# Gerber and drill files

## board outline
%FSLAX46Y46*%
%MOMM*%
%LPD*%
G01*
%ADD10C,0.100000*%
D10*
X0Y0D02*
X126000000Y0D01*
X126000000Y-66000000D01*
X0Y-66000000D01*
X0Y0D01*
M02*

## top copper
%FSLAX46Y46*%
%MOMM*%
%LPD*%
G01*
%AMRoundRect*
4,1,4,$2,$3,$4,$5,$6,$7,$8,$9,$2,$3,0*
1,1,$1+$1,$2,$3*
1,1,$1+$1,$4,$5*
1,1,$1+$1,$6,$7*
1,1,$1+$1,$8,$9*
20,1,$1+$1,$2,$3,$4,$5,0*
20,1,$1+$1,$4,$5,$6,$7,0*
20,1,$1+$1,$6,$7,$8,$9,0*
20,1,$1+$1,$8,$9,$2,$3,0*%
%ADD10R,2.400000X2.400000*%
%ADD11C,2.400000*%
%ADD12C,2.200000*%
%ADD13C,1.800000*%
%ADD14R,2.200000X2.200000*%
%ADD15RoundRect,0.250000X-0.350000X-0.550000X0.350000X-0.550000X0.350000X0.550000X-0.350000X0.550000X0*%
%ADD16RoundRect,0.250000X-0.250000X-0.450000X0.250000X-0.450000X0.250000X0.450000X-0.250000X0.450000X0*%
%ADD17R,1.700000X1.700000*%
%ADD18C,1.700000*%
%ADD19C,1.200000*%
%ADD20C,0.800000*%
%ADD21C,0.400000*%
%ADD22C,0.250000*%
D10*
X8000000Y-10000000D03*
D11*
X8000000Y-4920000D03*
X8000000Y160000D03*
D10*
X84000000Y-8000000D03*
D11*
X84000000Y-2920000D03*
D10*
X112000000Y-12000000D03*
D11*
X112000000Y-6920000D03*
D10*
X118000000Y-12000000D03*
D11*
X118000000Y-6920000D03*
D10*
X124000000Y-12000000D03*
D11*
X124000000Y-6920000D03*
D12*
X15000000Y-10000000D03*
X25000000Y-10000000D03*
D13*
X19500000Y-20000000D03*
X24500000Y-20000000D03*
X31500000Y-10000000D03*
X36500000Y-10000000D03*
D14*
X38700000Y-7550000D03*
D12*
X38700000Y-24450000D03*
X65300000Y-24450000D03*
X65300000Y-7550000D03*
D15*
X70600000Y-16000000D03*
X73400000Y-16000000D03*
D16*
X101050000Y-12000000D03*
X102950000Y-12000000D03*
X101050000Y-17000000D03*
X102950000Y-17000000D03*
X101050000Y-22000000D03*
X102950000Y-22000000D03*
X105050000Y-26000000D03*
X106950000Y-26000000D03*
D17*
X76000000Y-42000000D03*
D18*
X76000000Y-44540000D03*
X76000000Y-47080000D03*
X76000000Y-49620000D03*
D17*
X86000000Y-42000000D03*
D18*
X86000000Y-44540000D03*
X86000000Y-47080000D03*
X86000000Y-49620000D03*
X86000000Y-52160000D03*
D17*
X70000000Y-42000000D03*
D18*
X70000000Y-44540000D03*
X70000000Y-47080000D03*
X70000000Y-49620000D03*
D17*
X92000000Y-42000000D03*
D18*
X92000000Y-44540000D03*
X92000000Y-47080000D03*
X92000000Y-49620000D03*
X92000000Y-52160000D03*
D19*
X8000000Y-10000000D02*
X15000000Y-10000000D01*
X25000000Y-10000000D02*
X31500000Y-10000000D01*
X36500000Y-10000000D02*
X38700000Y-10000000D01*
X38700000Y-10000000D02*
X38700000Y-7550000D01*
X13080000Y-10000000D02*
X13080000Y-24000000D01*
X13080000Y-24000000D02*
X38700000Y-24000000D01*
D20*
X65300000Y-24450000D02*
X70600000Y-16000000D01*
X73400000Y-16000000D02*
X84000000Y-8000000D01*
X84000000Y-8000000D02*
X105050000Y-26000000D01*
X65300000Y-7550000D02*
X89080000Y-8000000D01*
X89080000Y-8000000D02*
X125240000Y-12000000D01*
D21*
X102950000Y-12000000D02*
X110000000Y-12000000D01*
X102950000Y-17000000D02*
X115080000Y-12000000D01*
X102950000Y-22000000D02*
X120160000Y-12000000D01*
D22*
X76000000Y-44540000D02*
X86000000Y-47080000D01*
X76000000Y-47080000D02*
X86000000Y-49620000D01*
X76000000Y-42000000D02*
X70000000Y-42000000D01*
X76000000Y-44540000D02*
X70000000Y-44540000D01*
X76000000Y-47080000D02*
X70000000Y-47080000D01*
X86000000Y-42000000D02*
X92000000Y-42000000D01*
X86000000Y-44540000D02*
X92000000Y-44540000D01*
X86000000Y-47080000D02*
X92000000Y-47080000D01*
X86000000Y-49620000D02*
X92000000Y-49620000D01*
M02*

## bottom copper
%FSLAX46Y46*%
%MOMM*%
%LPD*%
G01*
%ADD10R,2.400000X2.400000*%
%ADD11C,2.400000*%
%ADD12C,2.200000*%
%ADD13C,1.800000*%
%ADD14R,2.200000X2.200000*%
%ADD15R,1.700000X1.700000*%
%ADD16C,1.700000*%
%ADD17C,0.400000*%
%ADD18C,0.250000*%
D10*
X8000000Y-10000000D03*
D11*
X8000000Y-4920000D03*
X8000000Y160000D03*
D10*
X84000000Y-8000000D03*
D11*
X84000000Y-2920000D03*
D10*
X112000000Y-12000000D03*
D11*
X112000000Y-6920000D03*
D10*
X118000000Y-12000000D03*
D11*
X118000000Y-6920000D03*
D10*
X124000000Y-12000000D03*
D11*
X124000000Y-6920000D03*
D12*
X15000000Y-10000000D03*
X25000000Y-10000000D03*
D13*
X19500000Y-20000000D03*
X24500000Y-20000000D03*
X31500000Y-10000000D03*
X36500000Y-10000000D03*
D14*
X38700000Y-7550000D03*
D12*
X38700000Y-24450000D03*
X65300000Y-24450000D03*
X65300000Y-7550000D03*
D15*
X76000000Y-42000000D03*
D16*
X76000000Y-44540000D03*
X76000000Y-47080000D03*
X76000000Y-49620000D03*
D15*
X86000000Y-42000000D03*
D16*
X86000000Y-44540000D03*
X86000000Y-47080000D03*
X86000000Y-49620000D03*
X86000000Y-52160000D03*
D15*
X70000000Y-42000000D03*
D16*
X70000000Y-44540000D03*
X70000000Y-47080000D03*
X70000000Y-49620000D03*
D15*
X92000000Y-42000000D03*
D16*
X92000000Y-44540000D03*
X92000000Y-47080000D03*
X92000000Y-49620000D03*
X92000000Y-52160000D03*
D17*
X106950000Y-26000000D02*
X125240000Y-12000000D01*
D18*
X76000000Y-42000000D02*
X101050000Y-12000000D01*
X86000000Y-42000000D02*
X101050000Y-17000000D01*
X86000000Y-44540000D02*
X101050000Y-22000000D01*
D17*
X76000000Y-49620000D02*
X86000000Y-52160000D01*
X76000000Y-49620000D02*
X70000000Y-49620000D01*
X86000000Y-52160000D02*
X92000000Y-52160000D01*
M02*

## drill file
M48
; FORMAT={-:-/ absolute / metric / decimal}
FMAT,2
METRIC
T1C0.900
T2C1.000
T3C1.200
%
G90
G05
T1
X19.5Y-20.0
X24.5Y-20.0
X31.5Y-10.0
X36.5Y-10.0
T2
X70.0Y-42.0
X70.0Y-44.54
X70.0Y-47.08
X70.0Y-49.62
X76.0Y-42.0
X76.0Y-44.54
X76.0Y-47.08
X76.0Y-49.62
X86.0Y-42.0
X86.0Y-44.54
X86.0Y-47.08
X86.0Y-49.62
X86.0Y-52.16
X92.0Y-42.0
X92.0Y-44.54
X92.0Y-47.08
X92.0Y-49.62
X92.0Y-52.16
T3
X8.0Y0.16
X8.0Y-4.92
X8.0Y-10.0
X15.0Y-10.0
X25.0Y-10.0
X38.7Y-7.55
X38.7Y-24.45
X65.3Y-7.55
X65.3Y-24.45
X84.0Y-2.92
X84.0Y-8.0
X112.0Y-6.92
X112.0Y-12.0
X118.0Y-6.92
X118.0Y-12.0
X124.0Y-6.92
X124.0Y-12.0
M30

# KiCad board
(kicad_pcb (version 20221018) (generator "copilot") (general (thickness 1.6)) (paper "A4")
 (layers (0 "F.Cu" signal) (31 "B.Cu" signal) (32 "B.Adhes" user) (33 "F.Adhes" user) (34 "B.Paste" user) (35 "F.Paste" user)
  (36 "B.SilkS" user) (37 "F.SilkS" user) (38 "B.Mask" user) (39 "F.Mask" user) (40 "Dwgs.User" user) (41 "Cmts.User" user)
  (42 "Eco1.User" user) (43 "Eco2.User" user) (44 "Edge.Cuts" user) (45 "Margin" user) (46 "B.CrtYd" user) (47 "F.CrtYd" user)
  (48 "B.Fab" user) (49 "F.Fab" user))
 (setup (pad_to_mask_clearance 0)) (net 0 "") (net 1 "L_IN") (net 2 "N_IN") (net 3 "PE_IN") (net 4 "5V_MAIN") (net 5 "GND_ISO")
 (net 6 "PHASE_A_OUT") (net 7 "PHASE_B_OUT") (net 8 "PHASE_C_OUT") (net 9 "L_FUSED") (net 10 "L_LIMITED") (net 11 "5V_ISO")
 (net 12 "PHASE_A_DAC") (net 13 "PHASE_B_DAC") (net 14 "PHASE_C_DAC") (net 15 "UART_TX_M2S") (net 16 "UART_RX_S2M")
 (gr_rect (start 0 0) (end 126 66) (stroke (width 0.1) (type solid)) (fill none) (layer "Edge.Cuts"))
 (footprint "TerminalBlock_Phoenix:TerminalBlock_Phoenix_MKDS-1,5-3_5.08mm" (layer "F.Cu") (at 8 10 90)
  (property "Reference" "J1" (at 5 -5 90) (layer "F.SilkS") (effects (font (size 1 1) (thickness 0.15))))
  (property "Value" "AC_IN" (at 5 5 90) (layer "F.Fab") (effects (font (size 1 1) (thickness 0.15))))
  (pad "1" thru_hole rect (at 0 0 90) (size 2.4 2.4) (drill 1.2) (layers "*.Cu" "*.Mask") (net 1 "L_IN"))
  (pad "2" thru_hole circle (at 5.08 0 90) (size 2.4 2.4) (drill 1.2) (layers "*.Cu" "*.Mask") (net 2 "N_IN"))
  (pad "3" thru_hole circle (at 10.16 0 90) (size 2.4 2.4) (drill 1.2) (layers "*.Cu" "*.Mask") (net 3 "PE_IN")))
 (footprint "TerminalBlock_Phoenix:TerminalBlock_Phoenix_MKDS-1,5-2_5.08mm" (layer "F.Cu") (at 84 8 90)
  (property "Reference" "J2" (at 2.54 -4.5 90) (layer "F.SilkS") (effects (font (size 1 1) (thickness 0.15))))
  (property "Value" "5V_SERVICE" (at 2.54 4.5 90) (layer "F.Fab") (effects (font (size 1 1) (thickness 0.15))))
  (pad "1" thru_hole rect (at 0 0 90) (size 2.4 2.4) (drill 1.2) (layers "*.Cu" "*.Mask") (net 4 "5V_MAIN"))
  (pad "2" thru_hole circle (at 5.08 0 90) (size 2.4 2.4) (drill 1.2) (layers "*.Cu" "*.Mask") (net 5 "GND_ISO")))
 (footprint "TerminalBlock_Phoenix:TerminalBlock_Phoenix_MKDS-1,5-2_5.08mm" (layer "F.Cu") (at 112 12 90)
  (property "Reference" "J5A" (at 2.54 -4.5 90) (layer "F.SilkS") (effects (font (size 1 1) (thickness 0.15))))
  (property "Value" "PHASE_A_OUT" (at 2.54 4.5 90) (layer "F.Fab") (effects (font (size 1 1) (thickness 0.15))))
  (pad "1" thru_hole rect (at 0 0 90) (size 2.4 2.4) (drill 1.2) (layers "*.Cu" "*.Mask") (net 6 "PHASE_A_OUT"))
  (pad "2" thru_hole circle (at 5.08 0 90) (size 2.4 2.4) (drill 1.2) (layers "*.Cu" "*.Mask") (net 5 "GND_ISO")))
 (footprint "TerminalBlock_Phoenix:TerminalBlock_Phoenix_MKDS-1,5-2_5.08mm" (layer "F.Cu") (at 118 12 90)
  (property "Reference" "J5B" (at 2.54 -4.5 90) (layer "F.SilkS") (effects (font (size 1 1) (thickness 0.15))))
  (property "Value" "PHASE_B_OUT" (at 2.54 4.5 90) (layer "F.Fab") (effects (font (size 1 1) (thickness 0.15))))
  (pad "1" thru_hole rect (at 0 0 90) (size 2.4 2.4) (drill 1.2) (layers "*.Cu" "*.Mask") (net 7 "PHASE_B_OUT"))
  (pad "2" thru_hole circle (at 5.08 0 90) (size 2.4 2.4) (drill 1.2) (layers "*.Cu" "*.Mask") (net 5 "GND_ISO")))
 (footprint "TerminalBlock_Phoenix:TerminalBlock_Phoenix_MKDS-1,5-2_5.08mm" (layer "F.Cu") (at 124 12 90)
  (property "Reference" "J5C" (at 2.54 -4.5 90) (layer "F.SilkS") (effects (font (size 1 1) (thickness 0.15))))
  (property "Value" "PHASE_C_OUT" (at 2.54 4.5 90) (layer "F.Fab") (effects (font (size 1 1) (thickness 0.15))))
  (pad "1" thru_hole rect (at 0 0 90) (size 2.4 2.4) (drill 1.2) (layers "*.Cu" "*.Mask") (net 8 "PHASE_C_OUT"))
  (pad "2" thru_hole circle (at 5.08 0 90) (size 2.4 2.4) (drill 1.2) (layers "*.Cu" "*.Mask") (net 5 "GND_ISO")))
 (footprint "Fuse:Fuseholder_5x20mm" (layer "F.Cu") (at 20 10 0)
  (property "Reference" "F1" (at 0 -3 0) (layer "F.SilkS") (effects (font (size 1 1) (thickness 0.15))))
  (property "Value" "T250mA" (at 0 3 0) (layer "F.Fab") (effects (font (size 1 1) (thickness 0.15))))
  (pad "1" thru_hole circle (at -5 0 0) (size 2.2 2.2) (drill 1.2) (layers "*.Cu" "*.Mask") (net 1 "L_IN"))
  (pad "2" thru_hole circle (at 5 0 0) (size 2.2 2.2) (drill 1.2) (layers "*.Cu" "*.Mask") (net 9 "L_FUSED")))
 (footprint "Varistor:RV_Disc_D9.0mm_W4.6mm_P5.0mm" (layer "F.Cu") (at 22 20 0)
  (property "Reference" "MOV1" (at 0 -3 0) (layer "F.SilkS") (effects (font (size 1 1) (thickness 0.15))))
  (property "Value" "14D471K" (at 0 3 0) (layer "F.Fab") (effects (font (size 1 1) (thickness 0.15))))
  (pad "1" thru_hole circle (at -2.5 0 0) (size 1.8 1.8) (drill 0.9) (layers "*.Cu" "*.Mask") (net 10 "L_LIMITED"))
  (pad "2" thru_hole circle (at 2.5 0 0) (size 1.8 1.8) (drill 0.9) (layers "*.Cu" "*.Mask") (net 2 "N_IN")))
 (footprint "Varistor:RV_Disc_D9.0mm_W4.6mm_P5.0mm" (layer "F.Cu") (at 34 10 0)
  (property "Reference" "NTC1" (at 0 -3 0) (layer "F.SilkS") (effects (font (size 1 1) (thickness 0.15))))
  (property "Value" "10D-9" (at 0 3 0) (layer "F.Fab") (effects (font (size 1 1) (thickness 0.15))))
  (pad "1" thru_hole circle (at -2.5 0 0) (size 1.8 1.8) (drill 0.9) (layers "*.Cu" "*.Mask") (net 9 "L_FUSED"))
  (pad "2" thru_hole circle (at 2.5 0 0) (size 1.8 1.8) (drill 0.9) (layers "*.Cu" "*.Mask") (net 10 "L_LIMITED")))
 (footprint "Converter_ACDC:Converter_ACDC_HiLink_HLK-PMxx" (layer "F.Cu") (at 52 16 0)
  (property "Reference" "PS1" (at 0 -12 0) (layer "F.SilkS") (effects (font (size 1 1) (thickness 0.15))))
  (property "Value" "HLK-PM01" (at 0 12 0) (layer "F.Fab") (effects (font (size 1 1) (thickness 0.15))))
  (pad "1" thru_hole rect (at -13.3 -8.45 0) (size 2.2 2.2) (drill 1.2) (layers "*.Cu" "*.Mask") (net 10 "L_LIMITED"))
  (pad "2" thru_hole circle (at -13.3 8.45 0) (size 2.2 2.2) (drill 1.2) (layers "*.Cu" "*.Mask") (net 2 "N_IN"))
  (pad "3" thru_hole circle (at 13.3 8.45 0) (size 2.2 2.2) (drill 1.2) (layers "*.Cu" "*.Mask") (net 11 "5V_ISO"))
  (pad "4" thru_hole circle (at 13.3 -8.45 0) (size 2.2 2.2) (drill 1.2) (layers "*.Cu" "*.Mask") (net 5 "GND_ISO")))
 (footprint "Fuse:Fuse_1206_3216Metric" (layer "F.Cu") (at 72 16 0)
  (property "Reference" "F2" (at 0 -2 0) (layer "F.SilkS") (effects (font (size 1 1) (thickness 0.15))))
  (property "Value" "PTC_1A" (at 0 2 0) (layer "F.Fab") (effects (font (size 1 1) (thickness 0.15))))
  (pad "1" smd roundrect (at -1.4 0 0) (size 1.2 1.6) (layers "F.Cu" "F.Paste" "F.Mask") (roundrect_rratio 0.208333) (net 11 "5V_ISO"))
  (pad "2" smd roundrect (at 1.4 0 0) (size 1.2 1.6) (layers "F.Cu" "F.Paste" "F.Mask") (roundrect_rratio 0.208333) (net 4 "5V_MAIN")))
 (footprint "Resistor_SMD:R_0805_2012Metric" (layer "F.Cu") (at 102 12 0)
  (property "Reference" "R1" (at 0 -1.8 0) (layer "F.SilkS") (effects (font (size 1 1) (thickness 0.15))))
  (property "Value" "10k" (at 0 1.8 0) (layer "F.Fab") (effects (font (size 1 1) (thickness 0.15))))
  (pad "1" smd roundrect (at -0.95 0 0) (size 1 1.4) (layers "F.Cu" "F.Paste" "F.Mask") (roundrect_rratio 0.25) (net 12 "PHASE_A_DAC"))
  (pad "2" smd roundrect (at 0.95 0 0) (size 1 1.4) (layers "F.Cu" "F.Paste" "F.Mask") (roundrect_rratio 0.25) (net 6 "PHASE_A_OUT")))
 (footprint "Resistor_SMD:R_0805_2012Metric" (layer "F.Cu") (at 102 17 0)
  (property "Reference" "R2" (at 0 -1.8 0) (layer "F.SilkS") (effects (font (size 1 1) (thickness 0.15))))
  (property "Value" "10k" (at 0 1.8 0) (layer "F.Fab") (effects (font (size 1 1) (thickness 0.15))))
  (pad "1" smd roundrect (at -0.95 0 0) (size 1 1.4) (layers "F.Cu" "F.Paste" "F.Mask") (roundrect_rratio 0.25) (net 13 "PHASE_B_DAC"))
  (pad "2" smd roundrect (at 0.95 0 0) (size 1 1.4) (layers "F.Cu" "F.Paste" "F.Mask") (roundrect_rratio 0.25) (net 7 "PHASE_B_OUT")))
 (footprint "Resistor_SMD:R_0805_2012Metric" (layer "F.Cu") (at 102 22 0)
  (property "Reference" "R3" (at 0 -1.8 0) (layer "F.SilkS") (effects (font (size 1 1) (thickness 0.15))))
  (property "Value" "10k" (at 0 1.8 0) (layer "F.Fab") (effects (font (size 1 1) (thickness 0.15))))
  (pad "1" smd roundrect (at -0.95 0 0) (size 1 1.4) (layers "F.Cu" "F.Paste" "F.Mask") (roundrect_rratio 0.25) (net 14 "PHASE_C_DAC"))
  (pad "2" smd roundrect (at 0.95 0 0) (size 1 1.4) (layers "F.Cu" "F.Paste" "F.Mask") (roundrect_rratio 0.25) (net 8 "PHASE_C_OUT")))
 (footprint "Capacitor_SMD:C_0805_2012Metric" (layer "F.Cu") (at 106 26 0)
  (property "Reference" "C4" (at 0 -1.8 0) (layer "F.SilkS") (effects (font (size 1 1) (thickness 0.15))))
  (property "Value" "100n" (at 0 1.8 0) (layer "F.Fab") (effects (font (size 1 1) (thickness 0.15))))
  (pad "1" smd roundrect (at -0.95 0 0) (size 1 1.4) (layers "F.Cu" "F.Paste" "F.Mask") (roundrect_rratio 0.25) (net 4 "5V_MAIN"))
  (pad "2" smd roundrect (at 0.95 0 0) (size 1 1.4) (layers "F.Cu" "F.Paste" "F.Mask") (roundrect_rratio 0.25) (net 5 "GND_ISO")))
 (segment (start 8 10) (end 15 10) (width 1.2) (layer "F.Cu") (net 1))
 (segment (start 25 10) (end 31.5 10) (width 1.2) (layer "F.Cu") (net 9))
 (segment (start 36.5 10) (end 38.7 10) (width 1.2) (layer "F.Cu") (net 10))
 (segment (start 38.7 10) (end 38.7 7.55) (width 1.2) (layer "F.Cu") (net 10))
 (segment (start 13.08 10) (end 13.08 24) (width 1.2) (layer "F.Cu") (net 2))
 (segment (start 13.08 24) (end 38.7 24) (width 1.2) (layer "F.Cu") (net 2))
 (segment (start 65.3 24.45) (end 70.6 16) (width 0.8) (layer "F.Cu") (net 11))
 (segment (start 73.4 16) (end 84 8) (width 0.8) (layer "F.Cu") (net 4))
 (segment (start 84 8) (end 105.05 26) (width 0.8) (layer "F.Cu") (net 4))
 (segment (start 65.3 7.55) (end 89.08 8) (width 0.8) (layer "F.Cu") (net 5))
 (segment (start 89.08 8) (end 125.24 12) (width 0.8) (layer "F.Cu") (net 5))
 (segment (start 106.95 26) (end 125.24 12) (width 0.4) (layer "B.Cu") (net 5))
 (segment (start 102.95 12) (end 110 12) (width 0.4) (layer "F.Cu") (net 6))
 (segment (start 102.95 17) (end 115.08 12) (width 0.4) (layer "F.Cu") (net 7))
 (segment (start 102.95 22) (end 120.16 12) (width 0.4) (layer "F.Cu") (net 8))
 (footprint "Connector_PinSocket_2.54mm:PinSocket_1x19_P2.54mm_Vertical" (layer "F.Cu") (at 28 46 0)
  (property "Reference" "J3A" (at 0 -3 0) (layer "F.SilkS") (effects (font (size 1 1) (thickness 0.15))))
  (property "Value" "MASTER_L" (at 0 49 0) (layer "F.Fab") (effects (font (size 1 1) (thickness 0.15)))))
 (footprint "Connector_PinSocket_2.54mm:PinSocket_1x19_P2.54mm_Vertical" (layer "F.Cu") (at 36 46 0)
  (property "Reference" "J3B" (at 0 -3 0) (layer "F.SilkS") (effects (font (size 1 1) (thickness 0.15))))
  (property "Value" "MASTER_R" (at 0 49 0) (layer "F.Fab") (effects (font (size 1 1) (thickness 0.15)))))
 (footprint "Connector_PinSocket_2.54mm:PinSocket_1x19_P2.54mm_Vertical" (layer "F.Cu") (at 92 46 0)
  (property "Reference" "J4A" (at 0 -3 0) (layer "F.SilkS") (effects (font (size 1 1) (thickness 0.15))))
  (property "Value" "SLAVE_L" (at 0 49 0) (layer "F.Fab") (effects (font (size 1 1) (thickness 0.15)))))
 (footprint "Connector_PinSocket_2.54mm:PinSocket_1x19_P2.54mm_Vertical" (layer "F.Cu") (at 100 46 0)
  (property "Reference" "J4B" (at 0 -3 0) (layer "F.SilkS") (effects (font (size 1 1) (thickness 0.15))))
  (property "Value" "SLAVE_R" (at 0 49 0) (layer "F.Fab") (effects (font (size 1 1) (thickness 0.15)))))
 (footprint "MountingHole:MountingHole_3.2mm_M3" (layer "F.Cu") (at 5 5)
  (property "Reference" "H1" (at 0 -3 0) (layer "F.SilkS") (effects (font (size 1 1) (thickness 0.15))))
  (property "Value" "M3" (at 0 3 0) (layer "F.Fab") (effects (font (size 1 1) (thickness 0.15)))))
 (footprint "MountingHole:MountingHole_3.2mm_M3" (layer "F.Cu") (at 121 5)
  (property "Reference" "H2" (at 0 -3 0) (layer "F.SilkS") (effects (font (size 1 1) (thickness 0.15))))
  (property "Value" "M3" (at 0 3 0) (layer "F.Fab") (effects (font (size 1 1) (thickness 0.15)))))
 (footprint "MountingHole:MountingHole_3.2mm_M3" (layer "F.Cu") (at 5 61)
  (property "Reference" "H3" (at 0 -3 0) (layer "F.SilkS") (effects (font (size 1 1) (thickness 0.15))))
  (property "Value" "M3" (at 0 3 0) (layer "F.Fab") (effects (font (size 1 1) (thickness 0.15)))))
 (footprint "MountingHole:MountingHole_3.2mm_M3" (layer "F.Cu") (at 121 61)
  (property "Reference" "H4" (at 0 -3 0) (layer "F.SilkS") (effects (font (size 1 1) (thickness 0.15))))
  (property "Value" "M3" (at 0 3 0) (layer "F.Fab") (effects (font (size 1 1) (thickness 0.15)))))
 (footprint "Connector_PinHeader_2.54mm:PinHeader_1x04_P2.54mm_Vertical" (layer "F.Cu") (at 76 42 0)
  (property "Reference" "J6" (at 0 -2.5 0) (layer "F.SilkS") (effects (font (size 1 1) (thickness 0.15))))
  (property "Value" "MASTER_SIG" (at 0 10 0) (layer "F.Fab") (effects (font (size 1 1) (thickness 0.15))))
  (pad "1" thru_hole rect (at 0 0 0) (size 1.7 1.7) (drill 1) (layers "*.Cu" "*.Mask") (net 12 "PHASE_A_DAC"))
  (pad "2" thru_hole circle (at 0 2.54 0) (size 1.7 1.7) (drill 1) (layers "*.Cu" "*.Mask") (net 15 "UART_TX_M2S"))
  (pad "3" thru_hole circle (at 0 5.08 0) (size 1.7 1.7) (drill 1) (layers "*.Cu" "*.Mask") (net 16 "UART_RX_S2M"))
  (pad "4" thru_hole circle (at 0 7.62 0) (size 1.7 1.7) (drill 1) (layers "*.Cu" "*.Mask") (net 5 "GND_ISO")))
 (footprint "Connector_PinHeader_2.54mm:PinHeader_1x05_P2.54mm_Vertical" (layer "F.Cu") (at 86 42 0)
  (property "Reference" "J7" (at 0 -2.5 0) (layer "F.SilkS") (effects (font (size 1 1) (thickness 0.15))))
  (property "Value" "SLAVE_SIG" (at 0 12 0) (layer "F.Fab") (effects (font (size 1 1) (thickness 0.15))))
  (pad "1" thru_hole rect (at 0 0 0) (size 1.7 1.7) (drill 1) (layers "*.Cu" "*.Mask") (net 13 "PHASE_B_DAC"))
  (pad "2" thru_hole circle (at 0 2.54 0) (size 1.7 1.7) (drill 1) (layers "*.Cu" "*.Mask") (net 14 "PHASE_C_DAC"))
  (pad "3" thru_hole circle (at 0 5.08 0) (size 1.7 1.7) (drill 1) (layers "*.Cu" "*.Mask") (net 15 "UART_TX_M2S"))
  (pad "4" thru_hole circle (at 0 7.62 0) (size 1.7 1.7) (drill 1) (layers "*.Cu" "*.Mask") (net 16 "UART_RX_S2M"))
  (pad "5" thru_hole circle (at 0 10.16 0) (size 1.7 1.7) (drill 1) (layers "*.Cu" "*.Mask") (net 5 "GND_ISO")))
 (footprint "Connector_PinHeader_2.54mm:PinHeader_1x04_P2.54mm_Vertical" (layer "F.Cu") (at 70 42 0)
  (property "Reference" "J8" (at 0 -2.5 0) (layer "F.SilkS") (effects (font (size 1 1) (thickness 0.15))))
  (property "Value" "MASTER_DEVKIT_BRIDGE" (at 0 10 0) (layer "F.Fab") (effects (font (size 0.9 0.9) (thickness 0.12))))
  (pad "1" thru_hole rect (at 0 0 0) (size 1.7 1.7) (drill 1) (layers "*.Cu" "*.Mask") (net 12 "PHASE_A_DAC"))
  (pad "2" thru_hole circle (at 0 2.54 0) (size 1.7 1.7) (drill 1) (layers "*.Cu" "*.Mask") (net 15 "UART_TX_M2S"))
  (pad "3" thru_hole circle (at 0 5.08 0) (size 1.7 1.7) (drill 1) (layers "*.Cu" "*.Mask") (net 16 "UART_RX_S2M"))
  (pad "4" thru_hole circle (at 0 7.62 0) (size 1.7 1.7) (drill 1) (layers "*.Cu" "*.Mask") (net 5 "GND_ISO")))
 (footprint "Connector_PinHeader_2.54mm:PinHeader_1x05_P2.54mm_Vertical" (layer "F.Cu") (at 92 42 0)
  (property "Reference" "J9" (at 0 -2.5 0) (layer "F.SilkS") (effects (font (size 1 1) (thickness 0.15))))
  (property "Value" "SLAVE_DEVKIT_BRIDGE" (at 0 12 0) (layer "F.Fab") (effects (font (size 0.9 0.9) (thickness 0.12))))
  (pad "1" thru_hole rect (at 0 0 0) (size 1.7 1.7) (drill 1) (layers "*.Cu" "*.Mask") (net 13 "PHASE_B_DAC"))
  (pad "2" thru_hole circle (at 0 2.54 0) (size 1.7 1.7) (drill 1) (layers "*.Cu" "*.Mask") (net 14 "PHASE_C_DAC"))
  (pad "3" thru_hole circle (at 0 5.08 0) (size 1.7 1.7) (drill 1) (layers "*.Cu" "*.Mask") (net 15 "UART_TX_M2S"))
  (pad "4" thru_hole circle (at 0 7.62 0) (size 1.7 1.7) (drill 1) (layers "*.Cu" "*.Mask") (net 16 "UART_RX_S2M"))
  (pad "5" thru_hole circle (at 0 10.16 0) (size 1.7 1.7) (drill 1) (layers "*.Cu" "*.Mask") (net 5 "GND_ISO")))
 (segment (start 76 42) (end 101.05 12) (width 0.25) (layer "B.Cu") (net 12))
 (segment (start 86 42) (end 101.05 17) (width 0.25) (layer "B.Cu") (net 13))
 (segment (start 86 44.54) (end 101.05 22) (width 0.25) (layer "B.Cu") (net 14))
 (segment (start 76 44.54) (end 86 47.08) (width 0.25) (layer "F.Cu") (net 15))
 (segment (start 76 47.08) (end 86 49.62) (width 0.25) (layer "F.Cu") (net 16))
 (segment (start 76 49.62) (end 86 52.16) (width 0.4) (layer "B.Cu") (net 5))
 (segment (start 76 42) (end 70 42) (width 0.25) (layer "F.Cu") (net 12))
 (segment (start 76 44.54) (end 70 44.54) (width 0.25) (layer "F.Cu") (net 15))
 (segment (start 76 47.08) (end 70 47.08) (width 0.25) (layer "F.Cu") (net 16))
 (segment (start 76 49.62) (end 70 49.62) (width 0.4) (layer "B.Cu") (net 5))
 (segment (start 86 42) (end 92 42) (width 0.25) (layer "F.Cu") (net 13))
 (segment (start 86 44.54) (end 92 44.54) (width 0.25) (layer "F.Cu") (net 14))
 (segment (start 86 47.08) (end 92 47.08) (width 0.25) (layer "F.Cu") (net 15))
 (segment (start 86 49.62) (end 92 49.62) (width 0.25) (layer "F.Cu") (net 16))
 (segment (start 86 52.16) (end 92 52.16) (width 0.4) (layer "B.Cu") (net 5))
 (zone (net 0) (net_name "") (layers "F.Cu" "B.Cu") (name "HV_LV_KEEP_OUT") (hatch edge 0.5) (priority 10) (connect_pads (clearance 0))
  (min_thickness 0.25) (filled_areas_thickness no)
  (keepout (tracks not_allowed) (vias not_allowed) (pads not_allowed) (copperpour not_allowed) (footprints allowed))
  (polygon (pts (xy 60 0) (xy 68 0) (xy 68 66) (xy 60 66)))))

